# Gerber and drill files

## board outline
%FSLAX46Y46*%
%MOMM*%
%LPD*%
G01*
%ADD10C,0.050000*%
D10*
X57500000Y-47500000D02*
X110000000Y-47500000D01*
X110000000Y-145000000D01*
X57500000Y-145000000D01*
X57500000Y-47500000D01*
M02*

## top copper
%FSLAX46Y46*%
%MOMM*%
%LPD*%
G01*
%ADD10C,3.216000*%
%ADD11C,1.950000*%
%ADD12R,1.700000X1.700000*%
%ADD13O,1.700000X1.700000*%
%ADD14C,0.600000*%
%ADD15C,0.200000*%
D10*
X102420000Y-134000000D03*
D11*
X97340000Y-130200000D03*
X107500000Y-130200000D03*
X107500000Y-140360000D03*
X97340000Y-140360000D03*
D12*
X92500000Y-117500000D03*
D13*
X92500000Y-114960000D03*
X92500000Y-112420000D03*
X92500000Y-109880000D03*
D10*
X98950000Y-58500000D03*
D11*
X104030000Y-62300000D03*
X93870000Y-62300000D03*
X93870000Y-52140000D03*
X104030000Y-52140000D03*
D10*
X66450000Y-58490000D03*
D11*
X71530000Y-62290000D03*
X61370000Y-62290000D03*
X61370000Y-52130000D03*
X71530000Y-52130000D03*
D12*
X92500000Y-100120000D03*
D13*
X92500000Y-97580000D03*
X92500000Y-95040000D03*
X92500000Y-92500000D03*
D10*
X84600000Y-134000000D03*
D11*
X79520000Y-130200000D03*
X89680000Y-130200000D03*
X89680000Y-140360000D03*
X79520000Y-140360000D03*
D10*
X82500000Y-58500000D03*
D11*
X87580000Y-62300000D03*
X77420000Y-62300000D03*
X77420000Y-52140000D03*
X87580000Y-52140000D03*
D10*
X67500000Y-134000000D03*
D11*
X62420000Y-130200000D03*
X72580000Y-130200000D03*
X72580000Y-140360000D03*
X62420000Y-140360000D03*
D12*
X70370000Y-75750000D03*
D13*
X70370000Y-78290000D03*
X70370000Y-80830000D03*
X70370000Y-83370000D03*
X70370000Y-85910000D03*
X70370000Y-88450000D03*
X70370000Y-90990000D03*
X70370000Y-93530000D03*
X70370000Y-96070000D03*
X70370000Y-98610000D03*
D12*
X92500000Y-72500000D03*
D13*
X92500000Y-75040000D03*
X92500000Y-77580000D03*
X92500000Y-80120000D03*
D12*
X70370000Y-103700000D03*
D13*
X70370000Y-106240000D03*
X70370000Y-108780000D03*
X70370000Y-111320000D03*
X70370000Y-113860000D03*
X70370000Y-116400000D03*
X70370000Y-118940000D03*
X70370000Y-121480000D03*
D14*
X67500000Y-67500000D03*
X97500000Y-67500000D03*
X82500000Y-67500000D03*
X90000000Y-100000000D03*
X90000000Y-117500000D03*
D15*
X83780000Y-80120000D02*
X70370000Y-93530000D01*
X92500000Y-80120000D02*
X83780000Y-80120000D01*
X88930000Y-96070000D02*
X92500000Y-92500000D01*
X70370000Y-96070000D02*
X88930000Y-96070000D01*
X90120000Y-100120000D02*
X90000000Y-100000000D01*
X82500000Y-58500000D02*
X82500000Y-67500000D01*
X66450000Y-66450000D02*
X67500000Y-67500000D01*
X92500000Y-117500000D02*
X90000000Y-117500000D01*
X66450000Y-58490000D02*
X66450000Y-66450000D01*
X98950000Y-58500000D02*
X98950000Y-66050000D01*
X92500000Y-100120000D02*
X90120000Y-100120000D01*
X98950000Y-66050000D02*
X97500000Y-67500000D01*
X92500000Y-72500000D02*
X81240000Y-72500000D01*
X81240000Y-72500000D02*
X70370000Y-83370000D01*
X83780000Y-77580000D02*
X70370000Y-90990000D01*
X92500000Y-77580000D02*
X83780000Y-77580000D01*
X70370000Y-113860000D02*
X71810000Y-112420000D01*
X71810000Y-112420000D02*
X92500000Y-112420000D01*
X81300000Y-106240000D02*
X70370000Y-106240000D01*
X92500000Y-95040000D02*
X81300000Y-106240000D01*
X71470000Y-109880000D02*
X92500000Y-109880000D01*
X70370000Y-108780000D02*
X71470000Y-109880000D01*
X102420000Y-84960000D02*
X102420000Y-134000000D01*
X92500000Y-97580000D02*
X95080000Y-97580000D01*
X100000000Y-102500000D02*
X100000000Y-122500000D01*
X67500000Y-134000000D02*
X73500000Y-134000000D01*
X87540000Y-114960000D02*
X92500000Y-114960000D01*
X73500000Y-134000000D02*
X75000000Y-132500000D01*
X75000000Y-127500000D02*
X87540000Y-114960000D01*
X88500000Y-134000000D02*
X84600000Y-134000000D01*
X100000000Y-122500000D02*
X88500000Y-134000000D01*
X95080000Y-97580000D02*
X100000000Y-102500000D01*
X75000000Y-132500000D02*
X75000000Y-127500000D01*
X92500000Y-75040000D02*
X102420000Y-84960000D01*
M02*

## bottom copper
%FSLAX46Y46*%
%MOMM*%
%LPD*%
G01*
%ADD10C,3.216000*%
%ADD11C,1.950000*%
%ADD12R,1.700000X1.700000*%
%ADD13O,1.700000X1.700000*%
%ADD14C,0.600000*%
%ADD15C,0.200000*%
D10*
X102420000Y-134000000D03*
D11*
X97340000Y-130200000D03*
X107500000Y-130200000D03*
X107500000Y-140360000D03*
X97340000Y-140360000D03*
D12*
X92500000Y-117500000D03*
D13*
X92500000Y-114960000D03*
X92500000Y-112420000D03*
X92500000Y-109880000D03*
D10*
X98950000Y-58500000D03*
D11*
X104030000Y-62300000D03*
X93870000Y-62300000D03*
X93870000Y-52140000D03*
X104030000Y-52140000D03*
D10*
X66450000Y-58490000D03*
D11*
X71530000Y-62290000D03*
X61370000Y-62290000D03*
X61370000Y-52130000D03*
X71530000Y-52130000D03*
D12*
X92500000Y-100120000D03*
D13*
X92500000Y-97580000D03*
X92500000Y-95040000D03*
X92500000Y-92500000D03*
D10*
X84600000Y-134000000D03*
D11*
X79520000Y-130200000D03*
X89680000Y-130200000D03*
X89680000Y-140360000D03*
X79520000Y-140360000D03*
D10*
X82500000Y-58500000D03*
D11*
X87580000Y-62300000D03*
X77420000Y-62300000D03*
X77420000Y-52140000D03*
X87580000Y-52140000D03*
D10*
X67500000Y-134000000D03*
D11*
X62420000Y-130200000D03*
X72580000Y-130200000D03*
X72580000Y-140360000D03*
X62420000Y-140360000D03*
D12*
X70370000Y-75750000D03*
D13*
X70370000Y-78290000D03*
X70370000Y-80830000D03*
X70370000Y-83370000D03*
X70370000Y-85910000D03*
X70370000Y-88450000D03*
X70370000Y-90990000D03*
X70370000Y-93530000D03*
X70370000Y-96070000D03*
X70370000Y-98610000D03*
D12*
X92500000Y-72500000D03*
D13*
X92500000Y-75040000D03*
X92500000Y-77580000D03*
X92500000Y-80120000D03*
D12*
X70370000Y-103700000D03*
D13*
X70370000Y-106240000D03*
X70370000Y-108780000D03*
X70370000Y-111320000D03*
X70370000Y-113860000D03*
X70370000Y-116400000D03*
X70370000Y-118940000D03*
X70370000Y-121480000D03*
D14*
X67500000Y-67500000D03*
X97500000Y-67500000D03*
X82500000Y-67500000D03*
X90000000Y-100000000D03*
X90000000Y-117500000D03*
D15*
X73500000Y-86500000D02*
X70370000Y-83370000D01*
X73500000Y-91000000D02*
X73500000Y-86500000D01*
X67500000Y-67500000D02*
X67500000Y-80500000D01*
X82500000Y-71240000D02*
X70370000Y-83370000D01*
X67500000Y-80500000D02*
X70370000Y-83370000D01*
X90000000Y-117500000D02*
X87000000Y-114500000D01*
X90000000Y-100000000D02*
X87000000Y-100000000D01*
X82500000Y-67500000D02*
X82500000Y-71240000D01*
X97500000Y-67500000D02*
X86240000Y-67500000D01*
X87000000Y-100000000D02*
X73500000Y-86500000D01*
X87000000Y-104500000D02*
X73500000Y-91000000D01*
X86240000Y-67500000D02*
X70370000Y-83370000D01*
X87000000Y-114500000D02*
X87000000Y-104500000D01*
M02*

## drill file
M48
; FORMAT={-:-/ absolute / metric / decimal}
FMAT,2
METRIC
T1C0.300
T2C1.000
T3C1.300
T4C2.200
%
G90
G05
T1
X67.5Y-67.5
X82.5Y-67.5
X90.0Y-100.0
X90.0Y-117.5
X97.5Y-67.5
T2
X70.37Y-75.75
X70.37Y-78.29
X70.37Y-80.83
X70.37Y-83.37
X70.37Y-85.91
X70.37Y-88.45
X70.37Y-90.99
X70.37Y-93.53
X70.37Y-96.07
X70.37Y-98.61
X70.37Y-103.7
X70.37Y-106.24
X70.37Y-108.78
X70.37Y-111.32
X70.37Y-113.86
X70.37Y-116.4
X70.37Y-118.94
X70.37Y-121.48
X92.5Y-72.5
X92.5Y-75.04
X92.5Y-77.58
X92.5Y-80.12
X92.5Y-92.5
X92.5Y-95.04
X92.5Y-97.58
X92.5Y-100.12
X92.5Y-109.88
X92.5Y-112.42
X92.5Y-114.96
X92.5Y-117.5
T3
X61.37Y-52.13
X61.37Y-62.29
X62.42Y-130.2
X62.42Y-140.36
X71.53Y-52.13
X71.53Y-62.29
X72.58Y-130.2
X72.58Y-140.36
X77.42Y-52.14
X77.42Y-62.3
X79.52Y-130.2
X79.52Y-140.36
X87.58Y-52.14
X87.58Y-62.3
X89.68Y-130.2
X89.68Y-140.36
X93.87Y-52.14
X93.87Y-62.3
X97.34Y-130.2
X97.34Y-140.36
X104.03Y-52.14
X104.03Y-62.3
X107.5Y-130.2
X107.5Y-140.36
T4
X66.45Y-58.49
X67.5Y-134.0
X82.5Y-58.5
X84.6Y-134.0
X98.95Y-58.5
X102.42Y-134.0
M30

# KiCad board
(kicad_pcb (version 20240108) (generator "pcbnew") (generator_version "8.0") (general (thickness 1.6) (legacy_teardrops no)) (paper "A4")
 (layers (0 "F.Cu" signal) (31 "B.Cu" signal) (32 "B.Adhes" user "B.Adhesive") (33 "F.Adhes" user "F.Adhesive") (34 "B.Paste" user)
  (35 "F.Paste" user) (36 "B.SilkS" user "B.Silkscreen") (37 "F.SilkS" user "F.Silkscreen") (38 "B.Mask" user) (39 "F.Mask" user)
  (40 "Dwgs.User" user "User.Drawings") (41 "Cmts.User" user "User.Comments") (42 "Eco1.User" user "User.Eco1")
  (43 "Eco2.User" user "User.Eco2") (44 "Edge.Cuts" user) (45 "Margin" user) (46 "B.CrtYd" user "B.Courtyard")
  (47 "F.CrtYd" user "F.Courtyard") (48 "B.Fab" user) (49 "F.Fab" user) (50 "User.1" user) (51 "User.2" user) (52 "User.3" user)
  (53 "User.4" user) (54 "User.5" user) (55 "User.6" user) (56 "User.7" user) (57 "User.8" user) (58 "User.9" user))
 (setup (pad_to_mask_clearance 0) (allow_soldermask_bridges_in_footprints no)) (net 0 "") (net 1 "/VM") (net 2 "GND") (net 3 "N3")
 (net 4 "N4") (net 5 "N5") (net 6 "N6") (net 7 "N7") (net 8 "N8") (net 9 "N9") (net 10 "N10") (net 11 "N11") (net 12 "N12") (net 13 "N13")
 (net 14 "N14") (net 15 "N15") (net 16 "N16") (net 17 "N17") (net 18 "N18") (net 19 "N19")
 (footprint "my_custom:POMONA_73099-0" (layer "F.Cu") (at 102.42 134 -90)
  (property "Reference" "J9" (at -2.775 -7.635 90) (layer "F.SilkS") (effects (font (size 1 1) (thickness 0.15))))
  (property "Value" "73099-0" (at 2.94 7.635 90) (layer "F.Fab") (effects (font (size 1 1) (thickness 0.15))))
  (pad "1" thru_hole circle (at 0 0 270) (size 3.216 3.216) (drill 2.2) (layers "*.Cu" "*.Mask") (remove_unused_layers no) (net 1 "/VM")
   (solder_mask_margin 0.102))
  (pad "S1" thru_hole circle (at -3.8 5.08 270) (size 1.95 1.95) (drill 1.3) (layers "*.Cu" "*.Mask") (remove_unused_layers no)
   (solder_mask_margin 0.102))
  (pad "S2" thru_hole circle (at -3.8 -5.08 270) (size 1.95 1.95) (drill 1.3) (layers "*.Cu" "*.Mask") (remove_unused_layers no)
   (solder_mask_margin 0.102))
  (pad "S3" thru_hole circle (at 6.36 -5.08 270) (size 1.95 1.95) (drill 1.3) (layers "*.Cu" "*.Mask") (remove_unused_layers no)
   (solder_mask_margin 0.102))
  (pad "S4" thru_hole circle (at 6.36 5.08 270) (size 1.95 1.95) (drill 1.3) (layers "*.Cu" "*.Mask") (remove_unused_layers no)
   (solder_mask_margin 0.102)))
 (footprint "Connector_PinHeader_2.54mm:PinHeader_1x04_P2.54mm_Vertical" (layer "F.Cu") (at 92.5 117.5 180)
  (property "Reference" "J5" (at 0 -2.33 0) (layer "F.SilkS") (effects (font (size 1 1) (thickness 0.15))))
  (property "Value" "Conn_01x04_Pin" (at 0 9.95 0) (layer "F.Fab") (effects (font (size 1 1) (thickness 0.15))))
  (pad "1" thru_hole rect (at 0 0 180) (size 1.7 1.7) (drill 1) (layers "*.Cu" "*.Mask") (remove_unused_layers no) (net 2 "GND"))
  (pad "2" thru_hole oval (at 0 2.54 180) (size 1.7 1.7) (drill 1) (layers "*.Cu" "*.Mask") (remove_unused_layers no) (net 1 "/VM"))
  (pad "3" thru_hole oval (at 0 5.08 180) (size 1.7 1.7) (drill 1) (layers "*.Cu" "*.Mask") (remove_unused_layers no) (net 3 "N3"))
  (pad "4" thru_hole oval (at 0 7.62 180) (size 1.7 1.7) (drill 1) (layers "*.Cu" "*.Mask") (remove_unused_layers no) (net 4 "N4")))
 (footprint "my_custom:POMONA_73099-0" (layer "F.Cu") (at 98.95 58.5 90)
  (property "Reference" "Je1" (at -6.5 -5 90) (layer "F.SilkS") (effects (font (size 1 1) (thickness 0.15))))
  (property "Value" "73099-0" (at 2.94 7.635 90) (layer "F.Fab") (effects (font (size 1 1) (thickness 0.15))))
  (pad "1" thru_hole circle (at 0 0 90) (size 3.216 3.216) (drill 2.2) (layers "*.Cu" "*.Mask") (remove_unused_layers no) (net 2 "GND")
   (solder_mask_margin 0.102))
  (pad "S1" thru_hole circle (at -3.8 5.08 90) (size 1.95 1.95) (drill 1.3) (layers "*.Cu" "*.Mask") (remove_unused_layers no)
   (solder_mask_margin 0.102))
  (pad "S2" thru_hole circle (at -3.8 -5.08 90) (size 1.95 1.95) (drill 1.3) (layers "*.Cu" "*.Mask") (remove_unused_layers no)
   (solder_mask_margin 0.102))
  (pad "S3" thru_hole circle (at 6.36 -5.08 90) (size 1.95 1.95) (drill 1.3) (layers "*.Cu" "*.Mask") (remove_unused_layers no)
   (solder_mask_margin 0.102))
  (pad "S4" thru_hole circle (at 6.36 5.08 90) (size 1.95 1.95) (drill 1.3) (layers "*.Cu" "*.Mask") (remove_unused_layers no)
   (solder_mask_margin 0.102)))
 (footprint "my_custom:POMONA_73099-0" (layer "F.Cu") (at 66.45 58.49 90)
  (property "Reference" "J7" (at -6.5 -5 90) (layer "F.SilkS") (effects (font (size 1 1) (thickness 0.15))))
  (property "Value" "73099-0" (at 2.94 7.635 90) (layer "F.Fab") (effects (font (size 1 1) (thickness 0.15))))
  (pad "1" thru_hole circle (at 0 0 90) (size 3.216 3.216) (drill 2.2) (layers "*.Cu" "*.Mask") (remove_unused_layers no) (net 2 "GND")
   (solder_mask_margin 0.102))
  (pad "S1" thru_hole circle (at -3.8 5.08 90) (size 1.95 1.95) (drill 1.3) (layers "*.Cu" "*.Mask") (remove_unused_layers no)
   (solder_mask_margin 0.102))
  (pad "S2" thru_hole circle (at -3.8 -5.08 90) (size 1.95 1.95) (drill 1.3) (layers "*.Cu" "*.Mask") (remove_unused_layers no)
   (solder_mask_margin 0.102))
  (pad "S3" thru_hole circle (at 6.36 -5.08 90) (size 1.95 1.95) (drill 1.3) (layers "*.Cu" "*.Mask") (remove_unused_layers no)
   (solder_mask_margin 0.102))
  (pad "S4" thru_hole circle (at 6.36 5.08 90) (size 1.95 1.95) (drill 1.3) (layers "*.Cu" "*.Mask") (remove_unused_layers no)
   (solder_mask_margin 0.102)))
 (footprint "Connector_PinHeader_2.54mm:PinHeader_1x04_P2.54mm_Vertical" (layer "F.Cu") (at 92.5 100.12 180)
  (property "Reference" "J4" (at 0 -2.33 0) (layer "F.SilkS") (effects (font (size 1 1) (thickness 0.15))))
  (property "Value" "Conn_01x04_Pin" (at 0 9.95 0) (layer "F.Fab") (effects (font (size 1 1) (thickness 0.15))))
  (pad "1" thru_hole rect (at 0 0 180) (size 1.7 1.7) (drill 1) (layers "*.Cu" "*.Mask") (remove_unused_layers no) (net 2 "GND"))
  (pad "2" thru_hole oval (at 0 2.54 180) (size 1.7 1.7) (drill 1) (layers "*.Cu" "*.Mask") (remove_unused_layers no) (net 1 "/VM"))
  (pad "3" thru_hole oval (at 0 5.08 180) (size 1.7 1.7) (drill 1) (layers "*.Cu" "*.Mask") (remove_unused_layers no) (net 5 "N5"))
  (pad "4" thru_hole oval (at 0 7.62 180) (size 1.7 1.7) (drill 1) (layers "*.Cu" "*.Mask") (remove_unused_layers no) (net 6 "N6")))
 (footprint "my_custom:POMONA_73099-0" (layer "F.Cu") (at 84.6 134 -90)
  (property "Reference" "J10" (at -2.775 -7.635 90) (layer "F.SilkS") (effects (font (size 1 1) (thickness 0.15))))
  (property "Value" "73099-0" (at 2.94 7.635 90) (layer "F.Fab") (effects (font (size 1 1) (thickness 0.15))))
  (pad "1" thru_hole circle (at 0 0 270) (size 3.216 3.216) (drill 2.2) (layers "*.Cu" "*.Mask") (remove_unused_layers no) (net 1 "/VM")
   (solder_mask_margin 0.102))
  (pad "S1" thru_hole circle (at -3.8 5.08 270) (size 1.95 1.95) (drill 1.3) (layers "*.Cu" "*.Mask") (remove_unused_layers no)
   (solder_mask_margin 0.102))
  (pad "S2" thru_hole circle (at -3.8 -5.08 270) (size 1.95 1.95) (drill 1.3) (layers "*.Cu" "*.Mask") (remove_unused_layers no)
   (solder_mask_margin 0.102))
  (pad "S3" thru_hole circle (at 6.36 -5.08 270) (size 1.95 1.95) (drill 1.3) (layers "*.Cu" "*.Mask") (remove_unused_layers no)
   (solder_mask_margin 0.102))
  (pad "S4" thru_hole circle (at 6.36 5.08 270) (size 1.95 1.95) (drill 1.3) (layers "*.Cu" "*.Mask") (remove_unused_layers no)
   (solder_mask_margin 0.102)))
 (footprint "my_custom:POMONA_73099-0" (layer "F.Cu") (at 82.5 58.5 90)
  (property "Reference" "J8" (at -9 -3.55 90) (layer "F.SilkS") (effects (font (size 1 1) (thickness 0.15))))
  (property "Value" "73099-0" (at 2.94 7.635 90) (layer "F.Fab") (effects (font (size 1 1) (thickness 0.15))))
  (pad "1" thru_hole circle (at 0 0 90) (size 3.216 3.216) (drill 2.2) (layers "*.Cu" "*.Mask") (remove_unused_layers no) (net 2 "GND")
   (solder_mask_margin 0.102))
  (pad "S1" thru_hole circle (at -3.8 5.08 90) (size 1.95 1.95) (drill 1.3) (layers "*.Cu" "*.Mask") (remove_unused_layers no)
   (solder_mask_margin 0.102))
  (pad "S2" thru_hole circle (at -3.8 -5.08 90) (size 1.95 1.95) (drill 1.3) (layers "*.Cu" "*.Mask") (remove_unused_layers no)
   (solder_mask_margin 0.102))
  (pad "S3" thru_hole circle (at 6.36 -5.08 90) (size 1.95 1.95) (drill 1.3) (layers "*.Cu" "*.Mask") (remove_unused_layers no)
   (solder_mask_margin 0.102))
  (pad "S4" thru_hole circle (at 6.36 5.08 90) (size 1.95 1.95) (drill 1.3) (layers "*.Cu" "*.Mask") (remove_unused_layers no)
   (solder_mask_margin 0.102)))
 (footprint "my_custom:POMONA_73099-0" (layer "F.Cu") (at 67.5 134 -90)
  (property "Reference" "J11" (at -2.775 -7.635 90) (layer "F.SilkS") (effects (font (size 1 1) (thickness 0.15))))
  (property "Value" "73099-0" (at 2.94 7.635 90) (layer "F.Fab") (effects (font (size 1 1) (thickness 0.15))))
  (pad "1" thru_hole circle (at 0 0 270) (size 3.216 3.216) (drill 2.2) (layers "*.Cu" "*.Mask") (remove_unused_layers no) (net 1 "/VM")
   (solder_mask_margin 0.102))
  (pad "S1" thru_hole circle (at -3.8 5.08 270) (size 1.95 1.95) (drill 1.3) (layers "*.Cu" "*.Mask") (remove_unused_layers no)
   (solder_mask_margin 0.102))
  (pad "S2" thru_hole circle (at -3.8 -5.08 270) (size 1.95 1.95) (drill 1.3) (layers "*.Cu" "*.Mask") (remove_unused_layers no)
   (solder_mask_margin 0.102))
  (pad "S3" thru_hole circle (at 6.36 -5.08 270) (size 1.95 1.95) (drill 1.3) (layers "*.Cu" "*.Mask") (remove_unused_layers no)
   (solder_mask_margin 0.102))
  (pad "S4" thru_hole circle (at 6.36 5.08 270) (size 1.95 1.95) (drill 1.3) (layers "*.Cu" "*.Mask") (remove_unused_layers no)
   (solder_mask_margin 0.102)))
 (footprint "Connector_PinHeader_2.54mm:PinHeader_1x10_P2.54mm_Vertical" (layer "F.Cu") (at 70.37 75.75)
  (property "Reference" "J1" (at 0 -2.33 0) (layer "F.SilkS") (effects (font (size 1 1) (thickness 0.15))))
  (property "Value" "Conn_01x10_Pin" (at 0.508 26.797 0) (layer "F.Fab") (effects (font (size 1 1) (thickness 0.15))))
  (pad "1" thru_hole rect (at 0 0) (size 1.7 1.7) (drill 1) (layers "*.Cu" "*.Mask") (remove_unused_layers no) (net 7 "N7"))
  (pad "2" thru_hole oval (at 0 2.54) (size 1.7 1.7) (drill 1) (layers "*.Cu" "*.Mask") (remove_unused_layers no) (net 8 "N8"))
  (pad "3" thru_hole oval (at 0 5.08) (size 1.7 1.7) (drill 1) (layers "*.Cu" "*.Mask") (remove_unused_layers no) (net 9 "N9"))
  (pad "4" thru_hole oval (at 0 7.62) (size 1.7 1.7) (drill 1) (layers "*.Cu" "*.Mask") (remove_unused_layers no) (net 2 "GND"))
  (pad "5" thru_hole oval (at 0 10.16) (size 1.7 1.7) (drill 1) (layers "*.Cu" "*.Mask") (remove_unused_layers no) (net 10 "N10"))
  (pad "6" thru_hole oval (at 0 12.7) (size 1.7 1.7) (drill 1) (layers "*.Cu" "*.Mask") (remove_unused_layers no) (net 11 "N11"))
  (pad "7" thru_hole oval (at 0 15.24) (size 1.7 1.7) (drill 1) (layers "*.Cu" "*.Mask") (remove_unused_layers no) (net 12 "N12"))
  (pad "8" thru_hole oval (at 0 17.78) (size 1.7 1.7) (drill 1) (layers "*.Cu" "*.Mask") (remove_unused_layers no) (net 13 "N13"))
  (pad "9" thru_hole oval (at 0 20.32) (size 1.7 1.7) (drill 1) (layers "*.Cu" "*.Mask") (remove_unused_layers no) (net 6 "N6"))
  (pad "10" thru_hole oval (at 0 22.86) (size 1.7 1.7) (drill 1) (layers "*.Cu" "*.Mask") (remove_unused_layers no) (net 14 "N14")))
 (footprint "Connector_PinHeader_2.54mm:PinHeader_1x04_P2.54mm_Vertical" (layer "F.Cu") (at 92.5 72.5)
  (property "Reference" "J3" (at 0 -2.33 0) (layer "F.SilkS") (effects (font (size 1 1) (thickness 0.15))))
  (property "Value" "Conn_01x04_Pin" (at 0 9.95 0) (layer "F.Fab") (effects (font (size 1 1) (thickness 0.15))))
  (pad "1" thru_hole rect (at 0 0) (size 1.7 1.7) (drill 1) (layers "*.Cu" "*.Mask") (remove_unused_layers no) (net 2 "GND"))
  (pad "2" thru_hole oval (at 0 2.54) (size 1.7 1.7) (drill 1) (layers "*.Cu" "*.Mask") (remove_unused_layers no) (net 1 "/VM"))
  (pad "3" thru_hole oval (at 0 5.08) (size 1.7 1.7) (drill 1) (layers "*.Cu" "*.Mask") (remove_unused_layers no) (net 12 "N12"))
  (pad "4" thru_hole oval (at 0 7.62) (size 1.7 1.7) (drill 1) (layers "*.Cu" "*.Mask") (remove_unused_layers no) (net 13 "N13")))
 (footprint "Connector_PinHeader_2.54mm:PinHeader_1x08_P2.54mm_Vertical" (layer "F.Cu") (at 70.37 103.7)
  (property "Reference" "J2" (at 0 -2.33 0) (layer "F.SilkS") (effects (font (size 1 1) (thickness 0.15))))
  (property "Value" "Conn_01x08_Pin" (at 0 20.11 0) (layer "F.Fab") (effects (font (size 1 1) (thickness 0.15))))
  (pad "1" thru_hole rect (at 0 0) (size 1.7 1.7) (drill 1) (layers "*.Cu" "*.Mask") (remove_unused_layers no) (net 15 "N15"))
  (pad "2" thru_hole oval (at 0 2.54) (size 1.7 1.7) (drill 1) (layers "*.Cu" "*.Mask") (remove_unused_layers no) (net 5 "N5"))
  (pad "3" thru_hole oval (at 0 5.08) (size 1.7 1.7) (drill 1) (layers "*.Cu" "*.Mask") (remove_unused_layers no) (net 4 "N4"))
  (pad "4" thru_hole oval (at 0 7.62) (size 1.7 1.7) (drill 1) (layers "*.Cu" "*.Mask") (remove_unused_layers no) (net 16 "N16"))
  (pad "5" thru_hole oval (at 0 10.16) (size 1.7 1.7) (drill 1) (layers "*.Cu" "*.Mask") (remove_unused_layers no) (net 3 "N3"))
  (pad "6" thru_hole oval (at 0 12.7) (size 1.7 1.7) (drill 1) (layers "*.Cu" "*.Mask") (remove_unused_layers no) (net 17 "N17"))
  (pad "7" thru_hole oval (at 0 15.24) (size 1.7 1.7) (drill 1) (layers "*.Cu" "*.Mask") (remove_unused_layers no) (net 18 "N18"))
  (pad "8" thru_hole oval (at 0 17.78) (size 1.7 1.7) (drill 1) (layers "*.Cu" "*.Mask") (remove_unused_layers no) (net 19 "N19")))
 (gr_rect (start 57.5 47.5) (end 110 145) (stroke (width 0.05) (type default)) (fill none) (layer "Edge.Cuts"))
 (segment (start 83.78 80.12) (end 70.37 93.53) (width 0.2) (layer "F.Cu") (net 13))
 (segment (start 92.5 80.12) (end 83.78 80.12) (width 0.2) (layer "F.Cu") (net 13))
 (segment (start 88.93 96.07) (end 92.5 92.5) (width 0.2) (layer "F.Cu") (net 6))
 (segment (start 70.37 96.07) (end 88.93 96.07) (width 0.2) (layer "F.Cu") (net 6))
 (segment (start 90.12 100.12) (end 90 100) (width 0.2) (layer "F.Cu") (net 2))
 (segment (start 82.5 58.5) (end 82.5 67.5) (width 0.2) (layer "F.Cu") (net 2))
 (segment (start 66.45 66.45) (end 67.5 67.5) (width 0.2) (layer "F.Cu") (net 2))
 (segment (start 92.5 117.5) (end 90 117.5) (width 0.2) (layer "F.Cu") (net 2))
 (segment (start 66.45 58.49) (end 66.45 66.45) (width 0.2) (layer "F.Cu") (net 2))
 (segment (start 98.95 58.5) (end 98.95 66.05) (width 0.2) (layer "F.Cu") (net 2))
 (segment (start 92.5 100.12) (end 90.12 100.12) (width 0.2) (layer "F.Cu") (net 2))
 (segment (start 98.95 66.05) (end 97.5 67.5) (width 0.2) (layer "F.Cu") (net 2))
 (segment (start 92.5 72.5) (end 81.24 72.5) (width 0.2) (layer "F.Cu") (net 2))
 (segment (start 81.24 72.5) (end 70.37 83.37) (width 0.2) (layer "F.Cu") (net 2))
 (via (at 67.5 67.5) (size 0.6) (drill 0.3) (layers "F.Cu" "B.Cu") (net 2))
 (via (at 97.5 67.5) (size 0.6) (drill 0.3) (layers "F.Cu" "B.Cu") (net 2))
 (via (at 82.5 67.5) (size 0.6) (drill 0.3) (layers "F.Cu" "B.Cu") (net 2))
 (via (at 90 100) (size 0.6) (drill 0.3) (layers "F.Cu" "B.Cu") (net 2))
 (via (at 90 117.5) (size 0.6) (drill 0.3) (layers "F.Cu" "B.Cu") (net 2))
 (segment (start 73.5 86.5) (end 70.37 83.37) (width 0.2) (layer "B.Cu") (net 2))
 (segment (start 73.5 91) (end 73.5 86.5) (width 0.2) (layer "B.Cu") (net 2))
 (segment (start 67.5 67.5) (end 67.5 80.5) (width 0.2) (layer "B.Cu") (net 2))
 (segment (start 82.5 71.24) (end 70.37 83.37) (width 0.2) (layer "B.Cu") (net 2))
 (segment (start 67.5 80.5) (end 70.37 83.37) (width 0.2) (layer "B.Cu") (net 2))
 (segment (start 90 117.5) (end 87 114.5) (width 0.2) (layer "B.Cu") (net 2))
 (segment (start 90 100) (end 87 100) (width 0.2) (layer "B.Cu") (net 2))
 (segment (start 82.5 67.5) (end 82.5 71.24) (width 0.2) (layer "B.Cu") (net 2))
 (segment (start 97.5 67.5) (end 86.24 67.5) (width 0.2) (layer "B.Cu") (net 2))
 (segment (start 87 100) (end 73.5 86.5) (width 0.2) (layer "B.Cu") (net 2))
 (segment (start 87 104.5) (end 73.5 91) (width 0.2) (layer "B.Cu") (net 2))
 (segment (start 86.24 67.5) (end 70.37 83.37) (width 0.2) (layer "B.Cu") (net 2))
 (segment (start 87 114.5) (end 87 104.5) (width 0.2) (layer "B.Cu") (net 2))
 (segment (start 83.78 77.58) (end 70.37 90.99) (width 0.2) (layer "F.Cu") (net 12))
 (segment (start 92.5 77.58) (end 83.78 77.58) (width 0.2) (layer "F.Cu") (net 12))
 (segment (start 70.37 113.86) (end 71.81 112.42) (width 0.2) (layer "F.Cu") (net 3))
 (segment (start 71.81 112.42) (end 92.5 112.42) (width 0.2) (layer "F.Cu") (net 3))
 (segment (start 81.3 106.24) (end 70.37 106.24) (width 0.2) (layer "F.Cu") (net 5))
 (segment (start 92.5 95.04) (end 81.3 106.24) (width 0.2) (layer "F.Cu") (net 5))
 (segment (start 71.47 109.88) (end 92.5 109.88) (width 0.2) (layer "F.Cu") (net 4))
 (segment (start 70.37 108.78) (end 71.47 109.88) (width 0.2) (layer "F.Cu") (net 4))
 (segment (start 102.42 84.96) (end 102.42 134) (width 0.2) (layer "F.Cu") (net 1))
 (segment (start 92.5 97.58) (end 95.08 97.58) (width 0.2) (layer "F.Cu") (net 1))
 (segment (start 100 102.5) (end 100 122.5) (width 0.2) (layer "F.Cu") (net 1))
 (segment (start 67.5 134) (end 73.5 134) (width 0.2) (layer "F.Cu") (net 1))
 (segment (start 87.54 114.96) (end 92.5 114.96) (width 0.2) (layer "F.Cu") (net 1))
 (segment (start 73.5 134) (end 75 132.5) (width 0.2) (layer "F.Cu") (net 1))
 (segment (start 75 127.5) (end 87.54 114.96) (width 0.2) (layer "F.Cu") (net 1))
 (segment (start 88.5 134) (end 84.6 134) (width 0.2) (layer "F.Cu") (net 1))
 (segment (start 100 122.5) (end 88.5 134) (width 0.2) (layer "F.Cu") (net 1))
 (segment (start 95.08 97.58) (end 100 102.5) (width 0.2) (layer "F.Cu") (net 1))
 (segment (start 75 132.5) (end 75 127.5) (width 0.2) (layer "F.Cu") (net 1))
 (segment (start 92.5 75.04) (end 102.42 84.96) (width 0.2) (layer "F.Cu") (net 1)))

